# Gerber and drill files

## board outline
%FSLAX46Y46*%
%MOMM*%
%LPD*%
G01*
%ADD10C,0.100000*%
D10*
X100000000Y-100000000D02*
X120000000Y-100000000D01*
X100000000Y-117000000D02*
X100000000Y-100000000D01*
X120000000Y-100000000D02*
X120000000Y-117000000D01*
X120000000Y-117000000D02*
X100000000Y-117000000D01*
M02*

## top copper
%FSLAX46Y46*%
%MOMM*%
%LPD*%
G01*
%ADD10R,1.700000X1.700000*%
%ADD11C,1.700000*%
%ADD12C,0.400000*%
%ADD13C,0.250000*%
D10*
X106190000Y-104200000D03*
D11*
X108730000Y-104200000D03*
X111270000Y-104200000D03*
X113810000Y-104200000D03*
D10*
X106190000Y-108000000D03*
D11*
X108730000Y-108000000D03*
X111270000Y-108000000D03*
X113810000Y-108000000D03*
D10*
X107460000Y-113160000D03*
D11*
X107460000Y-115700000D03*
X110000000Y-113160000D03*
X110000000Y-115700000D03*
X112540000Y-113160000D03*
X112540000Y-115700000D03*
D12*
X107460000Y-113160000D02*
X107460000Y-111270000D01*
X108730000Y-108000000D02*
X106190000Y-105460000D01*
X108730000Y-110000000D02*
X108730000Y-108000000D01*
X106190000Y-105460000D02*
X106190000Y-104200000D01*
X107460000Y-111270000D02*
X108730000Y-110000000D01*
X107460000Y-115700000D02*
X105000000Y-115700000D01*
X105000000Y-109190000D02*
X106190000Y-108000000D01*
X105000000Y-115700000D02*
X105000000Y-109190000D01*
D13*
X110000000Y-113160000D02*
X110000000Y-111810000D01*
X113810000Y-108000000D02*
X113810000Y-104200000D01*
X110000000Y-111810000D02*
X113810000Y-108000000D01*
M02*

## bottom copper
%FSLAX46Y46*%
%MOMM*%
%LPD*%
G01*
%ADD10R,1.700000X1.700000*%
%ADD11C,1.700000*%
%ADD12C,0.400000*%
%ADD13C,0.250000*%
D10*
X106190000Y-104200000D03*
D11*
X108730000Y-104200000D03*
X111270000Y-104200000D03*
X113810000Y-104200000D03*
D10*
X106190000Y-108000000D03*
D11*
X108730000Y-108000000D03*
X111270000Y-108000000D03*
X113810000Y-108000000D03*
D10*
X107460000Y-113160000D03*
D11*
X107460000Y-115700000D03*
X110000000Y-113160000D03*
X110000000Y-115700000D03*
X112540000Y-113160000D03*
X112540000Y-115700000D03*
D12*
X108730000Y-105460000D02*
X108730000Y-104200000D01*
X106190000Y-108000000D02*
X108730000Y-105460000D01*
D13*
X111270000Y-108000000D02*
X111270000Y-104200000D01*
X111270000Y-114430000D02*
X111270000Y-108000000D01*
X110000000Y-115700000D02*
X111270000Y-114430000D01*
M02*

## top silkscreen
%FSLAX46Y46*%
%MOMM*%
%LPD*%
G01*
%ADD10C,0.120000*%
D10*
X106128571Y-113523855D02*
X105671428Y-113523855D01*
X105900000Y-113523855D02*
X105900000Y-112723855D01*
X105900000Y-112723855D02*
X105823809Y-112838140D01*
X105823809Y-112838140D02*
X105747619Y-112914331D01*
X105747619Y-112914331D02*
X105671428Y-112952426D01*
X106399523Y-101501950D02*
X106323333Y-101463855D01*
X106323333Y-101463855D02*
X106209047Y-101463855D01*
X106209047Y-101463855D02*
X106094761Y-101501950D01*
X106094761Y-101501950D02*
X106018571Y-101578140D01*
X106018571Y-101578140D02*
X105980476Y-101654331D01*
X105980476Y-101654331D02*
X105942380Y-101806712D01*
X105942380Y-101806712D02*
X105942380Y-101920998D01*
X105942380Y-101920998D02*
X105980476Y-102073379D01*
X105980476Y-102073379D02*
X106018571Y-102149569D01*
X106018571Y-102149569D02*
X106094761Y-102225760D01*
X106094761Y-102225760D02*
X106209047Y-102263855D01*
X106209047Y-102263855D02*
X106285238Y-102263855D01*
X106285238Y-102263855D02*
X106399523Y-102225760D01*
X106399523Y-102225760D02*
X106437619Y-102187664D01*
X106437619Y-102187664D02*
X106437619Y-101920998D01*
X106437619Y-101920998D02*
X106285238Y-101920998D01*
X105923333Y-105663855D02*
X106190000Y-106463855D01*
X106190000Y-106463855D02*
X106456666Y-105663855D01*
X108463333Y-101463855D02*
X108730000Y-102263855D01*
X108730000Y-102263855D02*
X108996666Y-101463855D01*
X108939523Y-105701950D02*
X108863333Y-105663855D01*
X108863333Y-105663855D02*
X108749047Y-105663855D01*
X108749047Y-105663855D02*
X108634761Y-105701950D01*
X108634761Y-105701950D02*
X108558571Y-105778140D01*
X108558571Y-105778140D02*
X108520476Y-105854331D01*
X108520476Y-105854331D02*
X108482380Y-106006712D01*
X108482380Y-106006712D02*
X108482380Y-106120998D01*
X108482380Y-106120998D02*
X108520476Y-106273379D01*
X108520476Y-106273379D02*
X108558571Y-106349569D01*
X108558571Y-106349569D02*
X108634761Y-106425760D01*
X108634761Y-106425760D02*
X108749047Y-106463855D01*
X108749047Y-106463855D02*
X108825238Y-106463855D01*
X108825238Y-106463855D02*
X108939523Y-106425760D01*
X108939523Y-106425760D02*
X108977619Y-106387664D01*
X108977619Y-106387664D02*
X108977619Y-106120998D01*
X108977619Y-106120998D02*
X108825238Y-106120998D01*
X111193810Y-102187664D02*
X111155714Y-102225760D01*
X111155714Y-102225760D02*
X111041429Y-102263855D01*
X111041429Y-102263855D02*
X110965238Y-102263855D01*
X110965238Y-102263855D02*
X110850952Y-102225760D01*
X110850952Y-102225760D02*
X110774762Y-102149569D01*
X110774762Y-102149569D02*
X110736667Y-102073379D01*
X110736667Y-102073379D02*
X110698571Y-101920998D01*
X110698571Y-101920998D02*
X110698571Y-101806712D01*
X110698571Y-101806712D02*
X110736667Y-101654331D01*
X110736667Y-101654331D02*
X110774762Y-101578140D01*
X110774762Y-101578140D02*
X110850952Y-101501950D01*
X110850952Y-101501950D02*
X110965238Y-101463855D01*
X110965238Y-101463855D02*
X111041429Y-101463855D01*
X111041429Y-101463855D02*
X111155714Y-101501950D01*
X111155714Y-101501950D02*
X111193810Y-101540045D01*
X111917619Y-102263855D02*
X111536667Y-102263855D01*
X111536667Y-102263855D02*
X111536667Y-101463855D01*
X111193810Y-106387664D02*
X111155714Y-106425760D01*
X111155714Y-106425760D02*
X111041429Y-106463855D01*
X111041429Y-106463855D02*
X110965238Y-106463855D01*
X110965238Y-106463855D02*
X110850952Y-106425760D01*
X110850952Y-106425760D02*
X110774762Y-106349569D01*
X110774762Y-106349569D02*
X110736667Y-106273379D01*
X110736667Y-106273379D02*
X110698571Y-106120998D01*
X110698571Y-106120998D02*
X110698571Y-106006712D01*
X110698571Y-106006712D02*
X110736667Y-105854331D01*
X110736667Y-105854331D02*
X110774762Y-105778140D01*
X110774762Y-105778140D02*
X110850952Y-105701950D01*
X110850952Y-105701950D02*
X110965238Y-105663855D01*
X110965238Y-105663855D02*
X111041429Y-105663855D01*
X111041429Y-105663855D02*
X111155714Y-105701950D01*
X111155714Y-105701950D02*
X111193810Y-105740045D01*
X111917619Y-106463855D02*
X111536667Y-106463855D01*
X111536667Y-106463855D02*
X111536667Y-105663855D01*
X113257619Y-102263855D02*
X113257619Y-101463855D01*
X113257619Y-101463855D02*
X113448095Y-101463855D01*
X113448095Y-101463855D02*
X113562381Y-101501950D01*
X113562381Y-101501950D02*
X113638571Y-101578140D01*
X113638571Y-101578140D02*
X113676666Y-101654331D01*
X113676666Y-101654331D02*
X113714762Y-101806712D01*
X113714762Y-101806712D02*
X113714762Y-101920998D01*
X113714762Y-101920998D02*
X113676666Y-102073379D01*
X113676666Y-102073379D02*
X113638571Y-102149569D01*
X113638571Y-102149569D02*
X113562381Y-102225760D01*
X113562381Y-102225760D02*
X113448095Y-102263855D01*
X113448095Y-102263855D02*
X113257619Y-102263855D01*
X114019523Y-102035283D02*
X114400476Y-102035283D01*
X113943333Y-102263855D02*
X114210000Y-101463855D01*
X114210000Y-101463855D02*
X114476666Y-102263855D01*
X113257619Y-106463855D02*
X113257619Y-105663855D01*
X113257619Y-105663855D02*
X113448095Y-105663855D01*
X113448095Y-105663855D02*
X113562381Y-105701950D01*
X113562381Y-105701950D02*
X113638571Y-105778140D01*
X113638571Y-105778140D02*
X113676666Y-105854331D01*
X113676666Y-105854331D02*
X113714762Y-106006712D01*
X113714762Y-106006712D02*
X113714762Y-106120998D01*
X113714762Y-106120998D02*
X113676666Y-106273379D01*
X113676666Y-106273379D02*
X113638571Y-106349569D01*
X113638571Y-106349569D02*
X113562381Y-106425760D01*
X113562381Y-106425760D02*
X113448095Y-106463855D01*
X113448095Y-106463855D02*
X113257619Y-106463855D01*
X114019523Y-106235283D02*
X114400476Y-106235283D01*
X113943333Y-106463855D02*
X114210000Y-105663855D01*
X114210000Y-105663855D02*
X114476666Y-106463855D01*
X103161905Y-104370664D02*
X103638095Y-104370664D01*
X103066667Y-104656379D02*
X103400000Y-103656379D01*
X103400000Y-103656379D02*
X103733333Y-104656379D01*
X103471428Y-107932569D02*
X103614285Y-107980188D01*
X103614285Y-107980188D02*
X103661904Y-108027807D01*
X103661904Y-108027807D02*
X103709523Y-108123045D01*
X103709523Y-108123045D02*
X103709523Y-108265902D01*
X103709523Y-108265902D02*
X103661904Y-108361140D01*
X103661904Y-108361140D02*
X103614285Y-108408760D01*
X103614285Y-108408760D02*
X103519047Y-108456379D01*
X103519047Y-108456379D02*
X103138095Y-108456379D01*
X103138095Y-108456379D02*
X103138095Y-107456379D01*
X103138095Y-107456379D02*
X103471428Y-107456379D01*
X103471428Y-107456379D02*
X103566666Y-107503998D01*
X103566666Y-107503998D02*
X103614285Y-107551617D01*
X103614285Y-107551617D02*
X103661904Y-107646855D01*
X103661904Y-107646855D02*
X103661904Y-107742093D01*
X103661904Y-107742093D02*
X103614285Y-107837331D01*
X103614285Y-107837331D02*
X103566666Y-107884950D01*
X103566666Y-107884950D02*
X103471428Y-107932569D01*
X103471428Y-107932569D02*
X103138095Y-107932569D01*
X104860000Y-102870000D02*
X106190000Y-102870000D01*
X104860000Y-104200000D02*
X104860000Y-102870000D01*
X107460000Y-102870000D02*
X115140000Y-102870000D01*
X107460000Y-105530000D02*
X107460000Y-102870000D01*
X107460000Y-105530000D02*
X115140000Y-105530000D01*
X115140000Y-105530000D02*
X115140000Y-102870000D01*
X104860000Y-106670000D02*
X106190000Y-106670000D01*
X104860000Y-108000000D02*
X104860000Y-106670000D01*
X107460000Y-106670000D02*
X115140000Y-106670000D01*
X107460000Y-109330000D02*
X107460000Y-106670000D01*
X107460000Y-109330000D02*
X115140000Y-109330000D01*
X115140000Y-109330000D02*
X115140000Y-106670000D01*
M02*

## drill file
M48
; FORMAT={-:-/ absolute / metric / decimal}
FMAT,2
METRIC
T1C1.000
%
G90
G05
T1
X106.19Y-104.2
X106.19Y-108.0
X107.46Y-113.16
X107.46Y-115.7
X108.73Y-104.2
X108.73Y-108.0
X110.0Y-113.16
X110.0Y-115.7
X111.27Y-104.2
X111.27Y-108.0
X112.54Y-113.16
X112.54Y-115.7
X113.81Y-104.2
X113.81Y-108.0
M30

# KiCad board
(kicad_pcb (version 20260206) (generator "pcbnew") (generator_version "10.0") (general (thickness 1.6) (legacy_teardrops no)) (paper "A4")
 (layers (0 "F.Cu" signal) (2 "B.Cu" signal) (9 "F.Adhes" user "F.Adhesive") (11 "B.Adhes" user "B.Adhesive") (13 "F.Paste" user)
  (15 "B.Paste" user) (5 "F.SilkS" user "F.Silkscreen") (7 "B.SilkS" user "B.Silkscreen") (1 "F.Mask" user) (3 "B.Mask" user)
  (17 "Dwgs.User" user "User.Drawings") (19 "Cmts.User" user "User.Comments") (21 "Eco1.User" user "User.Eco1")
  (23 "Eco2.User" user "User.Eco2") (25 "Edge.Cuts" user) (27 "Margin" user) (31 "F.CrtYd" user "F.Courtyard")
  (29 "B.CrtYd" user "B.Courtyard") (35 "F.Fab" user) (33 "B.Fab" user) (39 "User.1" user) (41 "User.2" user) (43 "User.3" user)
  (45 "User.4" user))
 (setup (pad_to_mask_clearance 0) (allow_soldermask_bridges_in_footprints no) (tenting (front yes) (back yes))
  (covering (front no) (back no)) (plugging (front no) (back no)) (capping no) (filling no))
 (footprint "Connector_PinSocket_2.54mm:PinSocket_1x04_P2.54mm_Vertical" (layer "F.Cu") (at 106.19 104.2 90)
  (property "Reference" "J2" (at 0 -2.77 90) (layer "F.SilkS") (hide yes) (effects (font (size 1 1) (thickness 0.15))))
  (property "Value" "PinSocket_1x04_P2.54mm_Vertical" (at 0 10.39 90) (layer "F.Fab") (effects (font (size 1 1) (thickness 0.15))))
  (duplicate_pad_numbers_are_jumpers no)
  (fp_line (start 1.33 -1.33) (end 1.33 0) (stroke (width 0.12) (type solid)) (layer "F.SilkS"))
  (fp_line (start 0 -1.33) (end 1.33 -1.33) (stroke (width 0.12) (type solid)) (layer "F.SilkS"))
  (fp_line (start 1.33 1.27) (end 1.33 8.95) (stroke (width 0.12) (type solid)) (layer "F.SilkS"))
  (fp_line (start -1.33 1.27) (end 1.33 1.27) (stroke (width 0.12) (type solid)) (layer "F.SilkS"))
  (fp_line (start -1.33 1.27) (end -1.33 8.95) (stroke (width 0.12) (type solid)) (layer "F.SilkS"))
  (fp_line (start -1.33 8.95) (end 1.33 8.95) (stroke (width 0.12) (type solid)) (layer "F.SilkS"))
  (pad "1" thru_hole rect (at 0 0 90) (size 1.7 1.7) (drill 1) (layers "*.Cu" "*.Mask") (remove_unused_layers no) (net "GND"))
  (pad "2" thru_hole circle (at 0 2.54 90) (size 1.7 1.7) (drill 1) (layers "*.Cu" "*.Mask") (remove_unused_layers no) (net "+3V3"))
  (pad "3" thru_hole circle (at 0 5.08 90) (size 1.7 1.7) (drill 1) (layers "*.Cu" "*.Mask") (remove_unused_layers no) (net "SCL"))
  (pad "4" thru_hole circle (at 0 7.62 90) (size 1.7 1.7) (drill 1) (layers "*.Cu" "*.Mask") (remove_unused_layers no) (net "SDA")))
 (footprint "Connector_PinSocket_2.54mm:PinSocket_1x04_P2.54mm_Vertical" (layer "F.Cu") (at 106.19 108 90)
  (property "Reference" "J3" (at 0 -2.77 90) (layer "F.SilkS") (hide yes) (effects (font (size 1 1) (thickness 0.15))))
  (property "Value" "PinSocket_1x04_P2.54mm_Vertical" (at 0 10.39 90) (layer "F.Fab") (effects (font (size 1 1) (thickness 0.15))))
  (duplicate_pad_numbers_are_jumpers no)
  (fp_line (start 1.33 -1.33) (end 1.33 0) (stroke (width 0.12) (type solid)) (layer "F.SilkS"))
  (fp_line (start 0 -1.33) (end 1.33 -1.33) (stroke (width 0.12) (type solid)) (layer "F.SilkS"))
  (fp_line (start 1.33 1.27) (end 1.33 8.95) (stroke (width 0.12) (type solid)) (layer "F.SilkS"))
  (fp_line (start -1.33 1.27) (end 1.33 1.27) (stroke (width 0.12) (type solid)) (layer "F.SilkS"))
  (fp_line (start -1.33 1.27) (end -1.33 8.95) (stroke (width 0.12) (type solid)) (layer "F.SilkS"))
  (fp_line (start -1.33 8.95) (end 1.33 8.95) (stroke (width 0.12) (type solid)) (layer "F.SilkS"))
  (pad "1" thru_hole rect (at 0 0 90) (size 1.7 1.7) (drill 1) (layers "*.Cu" "*.Mask") (remove_unused_layers no) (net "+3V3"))
  (pad "2" thru_hole circle (at 0 2.54 90) (size 1.7 1.7) (drill 1) (layers "*.Cu" "*.Mask") (remove_unused_layers no) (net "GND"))
  (pad "3" thru_hole circle (at 0 5.08 90) (size 1.7 1.7) (drill 1) (layers "*.Cu" "*.Mask") (remove_unused_layers no) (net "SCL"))
  (pad "4" thru_hole circle (at 0 7.62 90) (size 1.7 1.7) (drill 1) (layers "*.Cu" "*.Mask") (remove_unused_layers no) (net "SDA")))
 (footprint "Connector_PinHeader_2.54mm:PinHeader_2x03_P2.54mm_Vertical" (layer "B.Cu") (at 107.46 113.16 -90)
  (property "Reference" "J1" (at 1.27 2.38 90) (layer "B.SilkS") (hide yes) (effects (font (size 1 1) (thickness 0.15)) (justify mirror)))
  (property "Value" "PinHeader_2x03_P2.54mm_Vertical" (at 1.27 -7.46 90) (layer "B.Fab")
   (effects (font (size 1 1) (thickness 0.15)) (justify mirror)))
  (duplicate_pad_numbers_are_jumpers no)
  (pad "1" thru_hole rect (at 0 0 270) (size 1.7 1.7) (drill 1) (layers "*.Cu" "*.Mask") (remove_unused_layers no) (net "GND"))
  (pad "2" thru_hole circle (at 2.54 0 270) (size 1.7 1.7) (drill 1) (layers "*.Cu" "*.Mask") (remove_unused_layers no) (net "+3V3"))
  (pad "3" thru_hole circle (at 0 -2.54 270) (size 1.7 1.7) (drill 1) (layers "*.Cu" "*.Mask") (remove_unused_layers no) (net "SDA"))
  (pad "4" thru_hole circle (at 2.54 -2.54 270) (size 1.7 1.7) (drill 1) (layers "*.Cu" "*.Mask") (remove_unused_layers no) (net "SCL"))
  (pad "5" thru_hole circle (at 0 -5.08 270) (size 1.7 1.7) (drill 1) (layers "*.Cu" "*.Mask") (remove_unused_layers no))
  (pad "6" thru_hole circle (at 2.54 -5.08 270) (size 1.7 1.7) (drill 1) (layers "*.Cu" "*.Mask") (remove_unused_layers no)))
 (gr_line (start 100 100) (end 120 100) (stroke (width 0.1) (type default)) (layer "Edge.Cuts"))
 (gr_line (start 100 117) (end 100 100) (stroke (width 0.1) (type default)) (layer "Edge.Cuts"))
 (gr_line (start 120 100) (end 120 117) (stroke (width 0.1) (type default)) (layer "Edge.Cuts"))
 (gr_line (start 120 117) (end 100 117) (stroke (width 0.1) (type default)) (layer "Edge.Cuts"))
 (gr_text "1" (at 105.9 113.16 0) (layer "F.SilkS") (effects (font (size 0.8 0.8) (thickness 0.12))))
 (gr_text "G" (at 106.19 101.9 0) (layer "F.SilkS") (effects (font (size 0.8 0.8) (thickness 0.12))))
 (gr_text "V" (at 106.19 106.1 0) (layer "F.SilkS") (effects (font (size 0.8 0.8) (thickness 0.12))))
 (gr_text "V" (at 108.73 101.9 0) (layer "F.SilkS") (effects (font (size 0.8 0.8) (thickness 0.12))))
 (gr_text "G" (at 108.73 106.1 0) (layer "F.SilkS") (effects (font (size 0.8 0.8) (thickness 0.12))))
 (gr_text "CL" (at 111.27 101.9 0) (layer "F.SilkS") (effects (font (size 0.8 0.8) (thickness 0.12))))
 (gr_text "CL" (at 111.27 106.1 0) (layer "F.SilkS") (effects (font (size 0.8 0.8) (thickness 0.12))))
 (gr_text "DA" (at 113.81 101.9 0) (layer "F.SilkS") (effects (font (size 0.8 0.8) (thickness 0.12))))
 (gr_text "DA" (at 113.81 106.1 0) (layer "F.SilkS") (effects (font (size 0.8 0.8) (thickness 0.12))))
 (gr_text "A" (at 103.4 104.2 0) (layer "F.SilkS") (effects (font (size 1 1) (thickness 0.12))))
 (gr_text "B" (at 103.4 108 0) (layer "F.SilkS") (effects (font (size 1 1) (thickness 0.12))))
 (segment (start 107.46 113.16) (end 107.46 111.27) (width 0.4) (layer "F.Cu") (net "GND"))
 (segment (start 108.73 108) (end 106.19 105.46) (width 0.4) (layer "F.Cu") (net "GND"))
 (segment (start 108.73 110) (end 108.73 108) (width 0.4) (layer "F.Cu") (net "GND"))
 (segment (start 106.19 105.46) (end 106.19 104.2) (width 0.4) (layer "F.Cu") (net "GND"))
 (segment (start 107.46 111.27) (end 108.73 110) (width 0.4) (layer "F.Cu") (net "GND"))
 (segment (start 107.46 115.7) (end 105 115.7) (width 0.4) (layer "F.Cu") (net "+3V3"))
 (segment (start 105 109.19) (end 106.19 108) (width 0.4) (layer "F.Cu") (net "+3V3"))
 (segment (start 105 115.7) (end 105 109.19) (width 0.4) (layer "F.Cu") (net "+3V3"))
 (segment (start 108.73 105.46) (end 108.73 104.2) (width 0.4) (layer "B.Cu") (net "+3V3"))
 (segment (start 106.19 108) (end 108.73 105.46) (width 0.4) (layer "B.Cu") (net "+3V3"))
 (segment (start 110 113.16) (end 110 111.81) (width 0.25) (layer "F.Cu") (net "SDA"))
 (segment (start 113.81 108) (end 113.81 104.2) (width 0.25) (layer "F.Cu") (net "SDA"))
 (segment (start 110 111.81) (end 113.81 108) (width 0.25) (layer "F.Cu") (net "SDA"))
 (segment (start 111.27 108) (end 111.27 104.2) (width 0.25) (layer "B.Cu") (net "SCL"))
 (segment (start 111.27 114.43) (end 111.27 108) (width 0.25) (layer "B.Cu") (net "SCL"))
 (segment (start 110 115.7) (end 111.27 114.43) (width 0.25) (layer "B.Cu") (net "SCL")))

